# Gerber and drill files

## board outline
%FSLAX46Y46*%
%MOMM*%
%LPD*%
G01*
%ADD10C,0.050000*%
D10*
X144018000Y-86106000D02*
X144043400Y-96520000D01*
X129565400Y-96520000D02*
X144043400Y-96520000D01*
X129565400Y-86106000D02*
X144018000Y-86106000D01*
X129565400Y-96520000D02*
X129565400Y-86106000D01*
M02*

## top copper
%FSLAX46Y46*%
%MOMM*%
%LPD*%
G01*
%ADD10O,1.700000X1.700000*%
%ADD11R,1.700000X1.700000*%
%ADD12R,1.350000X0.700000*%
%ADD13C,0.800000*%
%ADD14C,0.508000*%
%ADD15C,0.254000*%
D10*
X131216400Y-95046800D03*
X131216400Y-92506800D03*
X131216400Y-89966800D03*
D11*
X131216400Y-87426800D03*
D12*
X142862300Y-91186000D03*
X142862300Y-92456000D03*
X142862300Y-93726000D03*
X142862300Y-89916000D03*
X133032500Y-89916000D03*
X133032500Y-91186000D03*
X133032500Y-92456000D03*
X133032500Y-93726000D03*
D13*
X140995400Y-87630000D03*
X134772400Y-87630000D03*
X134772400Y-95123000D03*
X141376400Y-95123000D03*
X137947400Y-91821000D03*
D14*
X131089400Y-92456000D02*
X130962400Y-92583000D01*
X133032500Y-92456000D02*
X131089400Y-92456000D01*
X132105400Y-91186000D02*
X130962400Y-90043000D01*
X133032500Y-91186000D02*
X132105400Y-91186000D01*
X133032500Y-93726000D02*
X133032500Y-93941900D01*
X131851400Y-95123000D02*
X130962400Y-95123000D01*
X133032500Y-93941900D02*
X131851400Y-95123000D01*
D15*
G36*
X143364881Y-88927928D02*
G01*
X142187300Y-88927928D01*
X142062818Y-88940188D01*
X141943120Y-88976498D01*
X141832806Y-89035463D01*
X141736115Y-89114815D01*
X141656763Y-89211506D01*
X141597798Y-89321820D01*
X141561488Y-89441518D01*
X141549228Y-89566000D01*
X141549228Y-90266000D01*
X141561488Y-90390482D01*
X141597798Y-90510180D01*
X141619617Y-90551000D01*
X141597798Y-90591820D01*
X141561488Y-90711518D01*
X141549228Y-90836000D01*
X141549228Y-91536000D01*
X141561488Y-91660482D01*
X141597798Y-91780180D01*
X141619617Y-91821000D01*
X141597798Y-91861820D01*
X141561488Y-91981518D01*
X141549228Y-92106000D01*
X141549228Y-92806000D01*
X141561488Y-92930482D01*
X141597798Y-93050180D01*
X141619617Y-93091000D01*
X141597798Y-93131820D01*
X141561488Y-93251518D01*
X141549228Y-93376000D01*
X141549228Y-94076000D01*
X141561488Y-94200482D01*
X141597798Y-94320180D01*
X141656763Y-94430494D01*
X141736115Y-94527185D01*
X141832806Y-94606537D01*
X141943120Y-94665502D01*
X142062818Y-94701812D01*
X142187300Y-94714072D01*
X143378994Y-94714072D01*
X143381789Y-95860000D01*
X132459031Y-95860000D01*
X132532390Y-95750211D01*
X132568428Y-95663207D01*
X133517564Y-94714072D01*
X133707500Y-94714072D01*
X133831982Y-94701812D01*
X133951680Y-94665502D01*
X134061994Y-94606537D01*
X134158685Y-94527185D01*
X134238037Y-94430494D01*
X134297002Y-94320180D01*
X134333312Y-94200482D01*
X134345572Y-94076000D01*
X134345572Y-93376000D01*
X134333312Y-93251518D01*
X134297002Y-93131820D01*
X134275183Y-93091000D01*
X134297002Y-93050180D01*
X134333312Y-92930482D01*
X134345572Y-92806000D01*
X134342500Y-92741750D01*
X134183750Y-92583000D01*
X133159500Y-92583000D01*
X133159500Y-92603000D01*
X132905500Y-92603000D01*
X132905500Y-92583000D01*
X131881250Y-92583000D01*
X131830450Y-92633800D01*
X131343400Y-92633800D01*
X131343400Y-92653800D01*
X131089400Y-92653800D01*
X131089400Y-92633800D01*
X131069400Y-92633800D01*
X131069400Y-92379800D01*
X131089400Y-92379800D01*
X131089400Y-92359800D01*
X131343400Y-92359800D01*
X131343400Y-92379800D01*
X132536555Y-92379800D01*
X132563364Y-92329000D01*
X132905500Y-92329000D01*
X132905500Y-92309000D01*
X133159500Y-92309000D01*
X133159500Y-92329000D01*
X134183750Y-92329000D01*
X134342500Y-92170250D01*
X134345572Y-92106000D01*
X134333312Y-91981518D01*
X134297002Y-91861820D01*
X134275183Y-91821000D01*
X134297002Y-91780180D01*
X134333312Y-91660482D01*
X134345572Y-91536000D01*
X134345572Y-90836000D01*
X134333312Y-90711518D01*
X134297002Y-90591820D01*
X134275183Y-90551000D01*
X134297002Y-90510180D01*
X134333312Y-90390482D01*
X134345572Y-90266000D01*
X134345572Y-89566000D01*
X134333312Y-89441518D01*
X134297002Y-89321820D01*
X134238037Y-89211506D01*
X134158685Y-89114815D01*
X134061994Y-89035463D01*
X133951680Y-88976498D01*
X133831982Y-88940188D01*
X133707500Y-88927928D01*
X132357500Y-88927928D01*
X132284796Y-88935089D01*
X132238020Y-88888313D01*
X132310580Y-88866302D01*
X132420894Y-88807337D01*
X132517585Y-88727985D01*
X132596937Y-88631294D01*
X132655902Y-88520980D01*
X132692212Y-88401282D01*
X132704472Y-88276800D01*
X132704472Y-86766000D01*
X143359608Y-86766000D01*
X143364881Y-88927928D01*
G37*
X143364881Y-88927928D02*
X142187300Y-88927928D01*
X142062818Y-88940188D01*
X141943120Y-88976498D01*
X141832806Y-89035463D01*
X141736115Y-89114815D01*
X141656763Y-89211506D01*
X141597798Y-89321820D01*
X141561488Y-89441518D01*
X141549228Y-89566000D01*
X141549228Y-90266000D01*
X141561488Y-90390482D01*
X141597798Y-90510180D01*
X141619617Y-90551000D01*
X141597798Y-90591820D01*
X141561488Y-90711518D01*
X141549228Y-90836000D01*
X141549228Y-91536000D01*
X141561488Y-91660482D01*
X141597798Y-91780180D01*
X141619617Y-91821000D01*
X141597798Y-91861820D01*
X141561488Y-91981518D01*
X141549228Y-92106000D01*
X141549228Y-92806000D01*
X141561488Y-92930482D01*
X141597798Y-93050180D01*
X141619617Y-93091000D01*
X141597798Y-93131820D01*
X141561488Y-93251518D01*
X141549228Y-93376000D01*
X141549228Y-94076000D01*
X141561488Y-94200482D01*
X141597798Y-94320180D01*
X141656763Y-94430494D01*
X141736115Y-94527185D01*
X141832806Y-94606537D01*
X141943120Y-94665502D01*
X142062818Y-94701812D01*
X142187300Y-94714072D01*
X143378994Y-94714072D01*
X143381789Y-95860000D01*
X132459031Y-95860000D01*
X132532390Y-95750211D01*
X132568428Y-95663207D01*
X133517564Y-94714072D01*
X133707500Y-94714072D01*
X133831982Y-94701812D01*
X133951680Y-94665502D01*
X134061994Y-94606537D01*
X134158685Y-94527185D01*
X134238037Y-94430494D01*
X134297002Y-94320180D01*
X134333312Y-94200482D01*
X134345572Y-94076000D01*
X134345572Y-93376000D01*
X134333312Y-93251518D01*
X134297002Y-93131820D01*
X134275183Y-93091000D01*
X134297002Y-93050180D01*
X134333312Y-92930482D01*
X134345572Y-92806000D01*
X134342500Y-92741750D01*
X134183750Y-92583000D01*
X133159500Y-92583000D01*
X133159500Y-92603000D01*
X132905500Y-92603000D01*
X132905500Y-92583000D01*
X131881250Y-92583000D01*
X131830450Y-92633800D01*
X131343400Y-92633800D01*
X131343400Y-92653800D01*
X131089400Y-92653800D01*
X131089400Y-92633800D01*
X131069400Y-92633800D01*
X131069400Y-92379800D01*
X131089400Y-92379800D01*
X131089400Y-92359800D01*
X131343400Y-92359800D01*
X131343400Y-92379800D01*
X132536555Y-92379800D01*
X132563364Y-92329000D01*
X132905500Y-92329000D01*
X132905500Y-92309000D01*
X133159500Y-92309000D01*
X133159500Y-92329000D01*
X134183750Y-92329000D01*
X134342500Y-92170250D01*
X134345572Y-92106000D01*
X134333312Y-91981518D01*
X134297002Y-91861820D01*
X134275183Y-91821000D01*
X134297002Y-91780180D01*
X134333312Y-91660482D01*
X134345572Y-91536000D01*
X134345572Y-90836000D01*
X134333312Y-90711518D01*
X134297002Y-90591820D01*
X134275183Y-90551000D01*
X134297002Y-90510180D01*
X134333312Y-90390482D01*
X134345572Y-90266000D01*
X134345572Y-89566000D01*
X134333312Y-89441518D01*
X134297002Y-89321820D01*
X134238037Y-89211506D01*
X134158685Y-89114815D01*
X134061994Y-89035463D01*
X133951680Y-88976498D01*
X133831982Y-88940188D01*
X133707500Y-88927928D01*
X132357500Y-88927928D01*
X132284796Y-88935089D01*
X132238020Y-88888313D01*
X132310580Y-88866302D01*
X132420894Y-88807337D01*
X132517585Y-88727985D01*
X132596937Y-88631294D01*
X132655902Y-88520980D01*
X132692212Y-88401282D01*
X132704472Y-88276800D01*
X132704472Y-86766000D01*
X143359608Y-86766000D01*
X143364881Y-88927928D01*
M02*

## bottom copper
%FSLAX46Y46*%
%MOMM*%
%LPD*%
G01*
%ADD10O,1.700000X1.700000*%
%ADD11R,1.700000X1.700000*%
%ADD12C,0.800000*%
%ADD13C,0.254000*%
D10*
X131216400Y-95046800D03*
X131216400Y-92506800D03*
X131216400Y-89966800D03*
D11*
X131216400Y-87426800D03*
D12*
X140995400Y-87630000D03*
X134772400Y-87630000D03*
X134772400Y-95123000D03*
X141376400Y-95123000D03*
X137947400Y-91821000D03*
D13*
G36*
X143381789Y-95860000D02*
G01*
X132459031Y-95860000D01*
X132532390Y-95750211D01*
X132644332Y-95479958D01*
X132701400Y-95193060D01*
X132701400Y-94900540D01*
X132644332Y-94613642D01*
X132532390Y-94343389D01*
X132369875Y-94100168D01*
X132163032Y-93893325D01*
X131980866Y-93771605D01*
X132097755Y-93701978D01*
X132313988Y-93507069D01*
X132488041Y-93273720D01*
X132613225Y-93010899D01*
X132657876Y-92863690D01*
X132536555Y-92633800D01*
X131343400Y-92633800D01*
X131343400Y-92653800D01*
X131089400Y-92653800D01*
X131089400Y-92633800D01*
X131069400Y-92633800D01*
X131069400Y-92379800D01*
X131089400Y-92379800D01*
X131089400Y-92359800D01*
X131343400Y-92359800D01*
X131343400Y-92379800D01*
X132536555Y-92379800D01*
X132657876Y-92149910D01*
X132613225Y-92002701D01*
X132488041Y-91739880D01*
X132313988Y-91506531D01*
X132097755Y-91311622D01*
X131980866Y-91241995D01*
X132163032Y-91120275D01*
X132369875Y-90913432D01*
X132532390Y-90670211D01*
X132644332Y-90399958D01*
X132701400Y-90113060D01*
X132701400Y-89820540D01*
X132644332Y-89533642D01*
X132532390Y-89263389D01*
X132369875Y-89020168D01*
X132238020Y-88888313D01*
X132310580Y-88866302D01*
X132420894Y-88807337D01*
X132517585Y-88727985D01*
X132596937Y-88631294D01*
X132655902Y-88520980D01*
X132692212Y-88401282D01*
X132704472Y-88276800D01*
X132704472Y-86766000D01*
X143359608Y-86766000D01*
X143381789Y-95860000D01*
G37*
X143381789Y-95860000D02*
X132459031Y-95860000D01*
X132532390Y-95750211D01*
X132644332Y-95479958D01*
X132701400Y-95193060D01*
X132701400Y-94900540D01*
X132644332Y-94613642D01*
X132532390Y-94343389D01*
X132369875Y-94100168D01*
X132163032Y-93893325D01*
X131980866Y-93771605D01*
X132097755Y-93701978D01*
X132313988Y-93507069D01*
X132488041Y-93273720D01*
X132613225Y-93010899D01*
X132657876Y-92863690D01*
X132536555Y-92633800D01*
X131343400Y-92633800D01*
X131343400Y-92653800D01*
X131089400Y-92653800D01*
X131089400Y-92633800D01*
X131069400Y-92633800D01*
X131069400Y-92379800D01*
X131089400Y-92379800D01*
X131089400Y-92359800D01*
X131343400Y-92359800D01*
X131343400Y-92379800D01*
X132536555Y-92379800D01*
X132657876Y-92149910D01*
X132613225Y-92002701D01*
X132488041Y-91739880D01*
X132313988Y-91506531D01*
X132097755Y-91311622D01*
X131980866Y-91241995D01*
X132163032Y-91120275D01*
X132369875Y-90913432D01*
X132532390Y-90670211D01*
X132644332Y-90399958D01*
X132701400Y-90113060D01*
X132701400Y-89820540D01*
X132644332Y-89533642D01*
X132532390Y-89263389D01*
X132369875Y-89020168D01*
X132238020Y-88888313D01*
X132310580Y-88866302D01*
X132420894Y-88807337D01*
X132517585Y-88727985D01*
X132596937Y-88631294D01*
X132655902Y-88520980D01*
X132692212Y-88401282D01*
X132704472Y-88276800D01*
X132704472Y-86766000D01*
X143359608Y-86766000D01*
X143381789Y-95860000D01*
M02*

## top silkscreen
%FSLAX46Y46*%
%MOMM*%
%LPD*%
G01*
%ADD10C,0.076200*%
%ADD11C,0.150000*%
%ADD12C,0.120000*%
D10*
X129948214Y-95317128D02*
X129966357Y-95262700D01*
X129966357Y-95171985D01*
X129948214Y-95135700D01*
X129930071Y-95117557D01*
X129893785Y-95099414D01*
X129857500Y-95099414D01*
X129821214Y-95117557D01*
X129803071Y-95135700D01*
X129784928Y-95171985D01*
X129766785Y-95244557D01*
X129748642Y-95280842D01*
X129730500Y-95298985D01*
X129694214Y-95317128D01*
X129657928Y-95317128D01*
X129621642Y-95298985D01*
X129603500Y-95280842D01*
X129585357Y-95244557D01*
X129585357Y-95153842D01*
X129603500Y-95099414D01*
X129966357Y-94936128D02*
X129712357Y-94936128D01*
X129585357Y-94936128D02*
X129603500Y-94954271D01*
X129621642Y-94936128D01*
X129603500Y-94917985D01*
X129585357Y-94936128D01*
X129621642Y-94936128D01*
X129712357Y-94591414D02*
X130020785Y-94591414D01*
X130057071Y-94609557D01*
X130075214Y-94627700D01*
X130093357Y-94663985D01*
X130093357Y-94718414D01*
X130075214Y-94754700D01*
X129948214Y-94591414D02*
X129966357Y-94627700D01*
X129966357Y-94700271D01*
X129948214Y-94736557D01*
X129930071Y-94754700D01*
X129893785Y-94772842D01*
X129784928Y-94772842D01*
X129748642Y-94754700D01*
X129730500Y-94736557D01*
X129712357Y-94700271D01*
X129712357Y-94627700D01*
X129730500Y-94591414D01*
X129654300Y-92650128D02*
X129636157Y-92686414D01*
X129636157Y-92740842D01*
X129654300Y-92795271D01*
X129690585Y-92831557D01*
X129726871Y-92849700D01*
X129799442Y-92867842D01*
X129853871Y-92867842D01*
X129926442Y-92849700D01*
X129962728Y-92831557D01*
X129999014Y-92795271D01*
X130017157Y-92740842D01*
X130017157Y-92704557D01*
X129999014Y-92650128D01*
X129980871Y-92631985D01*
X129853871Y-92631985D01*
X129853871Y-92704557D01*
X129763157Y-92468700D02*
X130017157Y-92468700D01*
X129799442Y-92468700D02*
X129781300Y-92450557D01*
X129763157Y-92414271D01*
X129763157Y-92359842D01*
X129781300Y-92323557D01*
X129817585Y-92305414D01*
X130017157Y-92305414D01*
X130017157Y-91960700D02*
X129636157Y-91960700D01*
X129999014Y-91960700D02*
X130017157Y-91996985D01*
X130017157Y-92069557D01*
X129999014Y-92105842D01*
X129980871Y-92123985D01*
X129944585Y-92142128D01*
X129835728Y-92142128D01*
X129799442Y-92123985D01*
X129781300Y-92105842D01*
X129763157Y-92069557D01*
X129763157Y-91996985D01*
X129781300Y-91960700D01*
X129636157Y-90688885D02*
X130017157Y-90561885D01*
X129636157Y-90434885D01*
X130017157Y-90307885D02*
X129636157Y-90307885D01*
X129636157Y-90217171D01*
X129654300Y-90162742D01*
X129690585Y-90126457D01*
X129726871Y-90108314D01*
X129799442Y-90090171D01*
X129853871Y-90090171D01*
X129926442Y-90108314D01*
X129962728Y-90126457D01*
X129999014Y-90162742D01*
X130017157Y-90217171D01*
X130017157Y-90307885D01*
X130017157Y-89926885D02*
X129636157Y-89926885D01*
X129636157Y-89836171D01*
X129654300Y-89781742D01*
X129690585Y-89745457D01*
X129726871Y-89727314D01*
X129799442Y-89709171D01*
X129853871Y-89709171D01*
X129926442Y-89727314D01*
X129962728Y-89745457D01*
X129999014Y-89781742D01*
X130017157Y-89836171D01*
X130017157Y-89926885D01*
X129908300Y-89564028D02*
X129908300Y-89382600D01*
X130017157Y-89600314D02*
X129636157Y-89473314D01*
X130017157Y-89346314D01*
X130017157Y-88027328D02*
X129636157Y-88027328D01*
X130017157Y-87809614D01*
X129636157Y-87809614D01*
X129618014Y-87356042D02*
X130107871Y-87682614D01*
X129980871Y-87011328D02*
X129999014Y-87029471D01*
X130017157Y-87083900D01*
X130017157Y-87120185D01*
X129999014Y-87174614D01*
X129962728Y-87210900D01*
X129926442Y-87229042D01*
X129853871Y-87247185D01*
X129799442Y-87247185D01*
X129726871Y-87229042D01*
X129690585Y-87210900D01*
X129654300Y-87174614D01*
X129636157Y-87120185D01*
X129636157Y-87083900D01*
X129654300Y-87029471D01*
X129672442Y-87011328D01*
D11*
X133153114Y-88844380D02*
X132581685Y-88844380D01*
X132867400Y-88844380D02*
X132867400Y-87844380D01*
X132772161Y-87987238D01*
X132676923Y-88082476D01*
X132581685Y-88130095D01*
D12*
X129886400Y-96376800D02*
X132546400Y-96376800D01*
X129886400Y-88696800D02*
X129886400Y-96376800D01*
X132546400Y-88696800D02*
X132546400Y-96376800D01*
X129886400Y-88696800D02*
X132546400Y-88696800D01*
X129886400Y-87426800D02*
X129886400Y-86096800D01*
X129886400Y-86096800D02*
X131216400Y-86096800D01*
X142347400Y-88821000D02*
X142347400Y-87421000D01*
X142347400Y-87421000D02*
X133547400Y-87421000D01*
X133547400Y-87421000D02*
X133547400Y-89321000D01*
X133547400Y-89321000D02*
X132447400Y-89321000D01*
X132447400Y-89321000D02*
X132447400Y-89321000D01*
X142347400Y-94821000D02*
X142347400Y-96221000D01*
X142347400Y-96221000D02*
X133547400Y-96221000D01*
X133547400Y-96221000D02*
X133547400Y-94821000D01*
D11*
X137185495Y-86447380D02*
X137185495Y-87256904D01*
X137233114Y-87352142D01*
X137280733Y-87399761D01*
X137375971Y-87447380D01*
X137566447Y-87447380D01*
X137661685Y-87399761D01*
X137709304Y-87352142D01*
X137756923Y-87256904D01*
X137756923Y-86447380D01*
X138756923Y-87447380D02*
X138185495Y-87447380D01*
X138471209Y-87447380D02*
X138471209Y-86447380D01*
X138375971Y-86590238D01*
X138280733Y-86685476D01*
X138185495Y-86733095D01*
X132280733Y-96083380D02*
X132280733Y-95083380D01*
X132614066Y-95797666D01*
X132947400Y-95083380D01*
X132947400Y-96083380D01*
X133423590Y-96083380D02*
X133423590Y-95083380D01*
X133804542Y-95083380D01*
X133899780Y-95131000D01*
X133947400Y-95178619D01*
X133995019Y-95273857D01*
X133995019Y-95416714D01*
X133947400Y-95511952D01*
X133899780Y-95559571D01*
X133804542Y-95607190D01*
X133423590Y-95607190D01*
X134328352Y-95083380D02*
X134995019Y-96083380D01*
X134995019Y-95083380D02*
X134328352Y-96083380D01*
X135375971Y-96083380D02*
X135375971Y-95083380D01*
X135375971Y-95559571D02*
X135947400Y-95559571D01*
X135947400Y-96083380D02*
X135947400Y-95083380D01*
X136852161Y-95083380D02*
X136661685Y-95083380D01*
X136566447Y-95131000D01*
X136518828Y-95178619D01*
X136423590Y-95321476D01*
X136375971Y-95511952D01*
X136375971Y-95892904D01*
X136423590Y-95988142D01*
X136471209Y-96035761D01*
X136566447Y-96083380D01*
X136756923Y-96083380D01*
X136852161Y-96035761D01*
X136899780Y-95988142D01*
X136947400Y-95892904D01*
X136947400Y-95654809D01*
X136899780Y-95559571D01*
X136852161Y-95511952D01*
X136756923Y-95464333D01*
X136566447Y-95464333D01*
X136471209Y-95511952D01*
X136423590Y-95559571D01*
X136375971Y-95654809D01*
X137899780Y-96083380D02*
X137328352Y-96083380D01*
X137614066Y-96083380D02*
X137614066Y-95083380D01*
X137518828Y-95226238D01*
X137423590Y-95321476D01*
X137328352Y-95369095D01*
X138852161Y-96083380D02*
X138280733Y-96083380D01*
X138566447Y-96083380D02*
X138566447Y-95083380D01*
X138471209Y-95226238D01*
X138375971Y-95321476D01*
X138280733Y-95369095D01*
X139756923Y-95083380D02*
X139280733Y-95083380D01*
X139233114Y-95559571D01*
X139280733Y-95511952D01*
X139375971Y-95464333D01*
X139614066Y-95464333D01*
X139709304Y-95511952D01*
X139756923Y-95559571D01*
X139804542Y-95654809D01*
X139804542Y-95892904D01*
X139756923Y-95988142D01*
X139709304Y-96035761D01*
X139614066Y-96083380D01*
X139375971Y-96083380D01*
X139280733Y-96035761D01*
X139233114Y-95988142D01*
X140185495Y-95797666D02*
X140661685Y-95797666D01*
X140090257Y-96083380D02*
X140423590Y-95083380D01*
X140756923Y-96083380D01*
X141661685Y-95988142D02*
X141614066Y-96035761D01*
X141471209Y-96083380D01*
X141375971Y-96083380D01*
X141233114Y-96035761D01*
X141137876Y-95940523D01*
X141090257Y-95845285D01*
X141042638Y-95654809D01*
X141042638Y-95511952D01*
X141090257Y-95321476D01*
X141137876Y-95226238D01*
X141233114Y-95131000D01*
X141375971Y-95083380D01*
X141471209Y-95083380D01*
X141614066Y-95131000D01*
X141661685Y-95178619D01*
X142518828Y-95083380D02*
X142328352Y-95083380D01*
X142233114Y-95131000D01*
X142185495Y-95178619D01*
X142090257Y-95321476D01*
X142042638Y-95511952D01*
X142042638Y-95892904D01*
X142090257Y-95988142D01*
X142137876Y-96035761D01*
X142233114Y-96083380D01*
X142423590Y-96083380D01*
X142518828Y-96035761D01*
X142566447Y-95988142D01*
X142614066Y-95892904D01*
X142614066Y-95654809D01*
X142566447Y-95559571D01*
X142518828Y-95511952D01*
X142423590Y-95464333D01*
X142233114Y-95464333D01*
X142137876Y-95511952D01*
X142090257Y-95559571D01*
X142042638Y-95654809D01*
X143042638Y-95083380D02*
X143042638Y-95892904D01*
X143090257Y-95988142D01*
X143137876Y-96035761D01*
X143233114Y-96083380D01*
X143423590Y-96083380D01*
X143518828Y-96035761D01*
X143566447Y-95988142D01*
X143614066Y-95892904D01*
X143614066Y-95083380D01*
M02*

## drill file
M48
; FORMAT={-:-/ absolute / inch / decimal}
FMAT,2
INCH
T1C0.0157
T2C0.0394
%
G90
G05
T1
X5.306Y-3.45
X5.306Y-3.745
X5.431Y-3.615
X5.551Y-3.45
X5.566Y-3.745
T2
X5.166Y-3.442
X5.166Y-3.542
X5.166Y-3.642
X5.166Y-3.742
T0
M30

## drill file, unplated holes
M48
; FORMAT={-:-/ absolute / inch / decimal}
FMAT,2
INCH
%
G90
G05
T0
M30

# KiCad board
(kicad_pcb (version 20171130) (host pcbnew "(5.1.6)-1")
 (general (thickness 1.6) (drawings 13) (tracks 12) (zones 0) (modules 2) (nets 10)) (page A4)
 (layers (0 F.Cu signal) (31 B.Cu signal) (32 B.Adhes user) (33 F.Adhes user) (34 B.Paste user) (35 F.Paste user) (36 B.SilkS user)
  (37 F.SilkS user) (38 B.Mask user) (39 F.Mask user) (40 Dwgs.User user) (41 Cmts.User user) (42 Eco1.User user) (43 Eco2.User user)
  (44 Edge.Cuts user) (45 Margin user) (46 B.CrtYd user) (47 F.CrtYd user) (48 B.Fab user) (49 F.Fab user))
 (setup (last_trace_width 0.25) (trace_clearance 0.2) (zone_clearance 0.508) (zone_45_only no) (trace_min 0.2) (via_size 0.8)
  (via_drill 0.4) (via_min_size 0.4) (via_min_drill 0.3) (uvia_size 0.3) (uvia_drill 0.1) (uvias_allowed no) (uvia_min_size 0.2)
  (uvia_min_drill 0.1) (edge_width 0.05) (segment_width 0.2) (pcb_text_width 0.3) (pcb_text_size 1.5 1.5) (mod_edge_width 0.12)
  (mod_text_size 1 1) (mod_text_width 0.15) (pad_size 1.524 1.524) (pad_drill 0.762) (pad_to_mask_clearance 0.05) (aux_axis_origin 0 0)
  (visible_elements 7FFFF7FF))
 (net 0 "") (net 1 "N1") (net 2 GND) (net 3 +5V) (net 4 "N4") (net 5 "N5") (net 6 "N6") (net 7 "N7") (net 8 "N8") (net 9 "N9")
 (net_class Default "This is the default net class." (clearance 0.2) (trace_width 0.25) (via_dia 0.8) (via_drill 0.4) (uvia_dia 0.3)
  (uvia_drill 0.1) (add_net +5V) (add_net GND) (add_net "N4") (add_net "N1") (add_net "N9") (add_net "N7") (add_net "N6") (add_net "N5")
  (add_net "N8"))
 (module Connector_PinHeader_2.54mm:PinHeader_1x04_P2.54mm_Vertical (layer F.Cu) (at 131.2164 87.4268)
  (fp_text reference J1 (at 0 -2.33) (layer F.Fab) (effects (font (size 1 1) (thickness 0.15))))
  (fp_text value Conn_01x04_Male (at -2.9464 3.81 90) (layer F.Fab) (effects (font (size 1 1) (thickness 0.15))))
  (fp_line (start -1.33 8.95) (end 1.33 8.95) (layer F.SilkS) (width 0.12))
  (fp_line (start -1.33 1.27) (end -1.33 8.95) (layer F.SilkS) (width 0.12))
  (fp_line (start 1.33 1.27) (end 1.33 8.95) (layer F.SilkS) (width 0.12))
  (fp_line (start -1.33 1.27) (end 1.33 1.27) (layer F.SilkS) (width 0.12))
  (fp_line (start -1.33 0) (end -1.33 -1.33) (layer F.SilkS) (width 0.12))
  (fp_line (start -1.33 -1.33) (end 0 -1.33) (layer F.SilkS) (width 0.12))
  (pad 4 thru_hole oval (at 0 7.62) (size 1.7 1.7) (drill 1) (layers *.Cu *.Mask) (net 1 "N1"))
  (pad 3 thru_hole oval (at 0 5.08) (size 1.7 1.7) (drill 1) (layers *.Cu *.Mask) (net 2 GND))
  (pad 2 thru_hole oval (at 0 2.54) (size 1.7 1.7) (drill 1) (layers *.Cu *.Mask) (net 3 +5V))
  (pad 1 thru_hole rect (at 0 0) (size 1.7 1.7) (drill 1) (layers *.Cu *.Mask) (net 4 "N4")))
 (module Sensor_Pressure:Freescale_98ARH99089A (layer F.Cu) (at 137.9474 91.821)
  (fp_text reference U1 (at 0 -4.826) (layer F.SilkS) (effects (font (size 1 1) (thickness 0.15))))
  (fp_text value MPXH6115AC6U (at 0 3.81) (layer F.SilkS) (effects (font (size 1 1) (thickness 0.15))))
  (fp_line (start 4.4 -3) (end 4.4 -4.4) (layer F.SilkS) (width 0.12))
  (fp_line (start 4.4 -4.4) (end -4.4 -4.4) (layer F.SilkS) (width 0.12))
  (fp_line (start -4.4 -4.4) (end -4.4 -2.5) (layer F.SilkS) (width 0.12))
  (fp_line (start -4.4 -2.5) (end -5.5 -2.5) (layer F.SilkS) (width 0.12))
  (fp_line (start -5.5 -2.5) (end -5.5 -2.5) (layer F.SilkS) (width 0.12))
  (fp_line (start 4.4 3) (end 4.4 4.4) (layer F.SilkS) (width 0.12))
  (fp_line (start 4.4 4.4) (end -4.4 4.4) (layer F.SilkS) (width 0.12))
  (fp_line (start -4.4 4.4) (end -4.4 3) (layer F.SilkS) (width 0.12))
  (pad 7 smd rect (at 4.9149 -0.635) (size 1.35 0.7) (layers F.Cu F.Paste F.Mask) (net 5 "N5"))
  (pad 6 smd rect (at 4.9149 0.635) (size 1.35 0.7) (layers F.Cu F.Paste F.Mask) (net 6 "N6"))
  (pad 5 smd rect (at 4.9149 1.905) (size 1.35 0.7) (layers F.Cu F.Paste F.Mask) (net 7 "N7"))
  (pad 8 smd rect (at 4.9149 -1.905) (size 1.35 0.7) (layers F.Cu F.Paste F.Mask) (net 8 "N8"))
  (pad 1 smd rect (at -4.9149 -1.905) (size 1.35 0.7) (layers F.Cu F.Paste F.Mask) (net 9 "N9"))
  (pad 2 smd rect (at -4.9149 -0.635) (size 1.35 0.7) (layers F.Cu F.Paste F.Mask) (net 3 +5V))
  (pad 3 smd rect (at -4.9149 0.635) (size 1.35 0.7) (layers F.Cu F.Paste F.Mask) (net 2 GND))
  (pad 4 smd rect (at -4.9149 1.905) (size 1.35 0.7) (layers F.Cu F.Paste F.Mask) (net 1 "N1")))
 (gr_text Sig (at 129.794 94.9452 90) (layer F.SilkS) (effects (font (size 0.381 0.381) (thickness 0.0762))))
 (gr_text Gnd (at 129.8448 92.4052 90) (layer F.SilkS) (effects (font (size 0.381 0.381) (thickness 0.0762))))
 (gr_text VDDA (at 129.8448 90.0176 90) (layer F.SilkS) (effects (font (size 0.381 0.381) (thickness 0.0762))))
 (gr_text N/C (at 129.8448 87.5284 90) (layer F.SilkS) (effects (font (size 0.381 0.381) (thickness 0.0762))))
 (gr_line (start 144.018 86.106) (end 144.0434 96.52) (layer Edge.Cuts) (width 0.05))
 (gr_line (start 129.5654 96.52) (end 144.0434 96.52) (layer Edge.Cuts) (width 0.05))
 (gr_line (start 129.5654 86.106) (end 144.018 86.106) (layer Edge.Cuts) (width 0.05))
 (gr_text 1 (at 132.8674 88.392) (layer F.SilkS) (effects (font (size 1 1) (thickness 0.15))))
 (gr_line (start 129.5654 96.52) (end 129.5654 86.106) (layer Edge.Cuts) (width 0.05))
 (via (at 140.9954 87.63) (size 0.8) (drill 0.4) (layers F.Cu B.Cu) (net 2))
 (via (at 134.7724 87.63) (size 0.8) (drill 0.4) (layers F.Cu B.Cu) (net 2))
 (via (at 134.7724 95.123) (size 0.8) (drill 0.4) (layers F.Cu B.Cu) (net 2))
 (via (at 141.3764 95.123) (size 0.8) (drill 0.4) (layers F.Cu B.Cu) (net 2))
 (via (at 137.9474 91.821) (size 0.8) (drill 0.4) (layers F.Cu B.Cu) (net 2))
 (segment (start 131.0894 92.456) (end 130.9624 92.583) (width 0.508) (layer F.Cu) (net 2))
 (segment (start 133.0325 92.456) (end 131.0894 92.456) (width 0.508) (layer F.Cu) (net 2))
 (segment (start 132.1054 91.186) (end 130.9624 90.043) (width 0.508) (layer F.Cu) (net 3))
 (segment (start 133.0325 91.186) (end 132.1054 91.186) (width 0.508) (layer F.Cu) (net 3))
 (segment (start 133.0325 93.726) (end 133.0325 93.9419) (width 0.508) (layer F.Cu) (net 1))
 (segment (start 131.8514 95.123) (end 130.9624 95.123) (width 0.508) (layer F.Cu) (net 1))
 (segment (start 133.0325 93.9419) (end 131.8514 95.123) (width 0.508) (layer F.Cu) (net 1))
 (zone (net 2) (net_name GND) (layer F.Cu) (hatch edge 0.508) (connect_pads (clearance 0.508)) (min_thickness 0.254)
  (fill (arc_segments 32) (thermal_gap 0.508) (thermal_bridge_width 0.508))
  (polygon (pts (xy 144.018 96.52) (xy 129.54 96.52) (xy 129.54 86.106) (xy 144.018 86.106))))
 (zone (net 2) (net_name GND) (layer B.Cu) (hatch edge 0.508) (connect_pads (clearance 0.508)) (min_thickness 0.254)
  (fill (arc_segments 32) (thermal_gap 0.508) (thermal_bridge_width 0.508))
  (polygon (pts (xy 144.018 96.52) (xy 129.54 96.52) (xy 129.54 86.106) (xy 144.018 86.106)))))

